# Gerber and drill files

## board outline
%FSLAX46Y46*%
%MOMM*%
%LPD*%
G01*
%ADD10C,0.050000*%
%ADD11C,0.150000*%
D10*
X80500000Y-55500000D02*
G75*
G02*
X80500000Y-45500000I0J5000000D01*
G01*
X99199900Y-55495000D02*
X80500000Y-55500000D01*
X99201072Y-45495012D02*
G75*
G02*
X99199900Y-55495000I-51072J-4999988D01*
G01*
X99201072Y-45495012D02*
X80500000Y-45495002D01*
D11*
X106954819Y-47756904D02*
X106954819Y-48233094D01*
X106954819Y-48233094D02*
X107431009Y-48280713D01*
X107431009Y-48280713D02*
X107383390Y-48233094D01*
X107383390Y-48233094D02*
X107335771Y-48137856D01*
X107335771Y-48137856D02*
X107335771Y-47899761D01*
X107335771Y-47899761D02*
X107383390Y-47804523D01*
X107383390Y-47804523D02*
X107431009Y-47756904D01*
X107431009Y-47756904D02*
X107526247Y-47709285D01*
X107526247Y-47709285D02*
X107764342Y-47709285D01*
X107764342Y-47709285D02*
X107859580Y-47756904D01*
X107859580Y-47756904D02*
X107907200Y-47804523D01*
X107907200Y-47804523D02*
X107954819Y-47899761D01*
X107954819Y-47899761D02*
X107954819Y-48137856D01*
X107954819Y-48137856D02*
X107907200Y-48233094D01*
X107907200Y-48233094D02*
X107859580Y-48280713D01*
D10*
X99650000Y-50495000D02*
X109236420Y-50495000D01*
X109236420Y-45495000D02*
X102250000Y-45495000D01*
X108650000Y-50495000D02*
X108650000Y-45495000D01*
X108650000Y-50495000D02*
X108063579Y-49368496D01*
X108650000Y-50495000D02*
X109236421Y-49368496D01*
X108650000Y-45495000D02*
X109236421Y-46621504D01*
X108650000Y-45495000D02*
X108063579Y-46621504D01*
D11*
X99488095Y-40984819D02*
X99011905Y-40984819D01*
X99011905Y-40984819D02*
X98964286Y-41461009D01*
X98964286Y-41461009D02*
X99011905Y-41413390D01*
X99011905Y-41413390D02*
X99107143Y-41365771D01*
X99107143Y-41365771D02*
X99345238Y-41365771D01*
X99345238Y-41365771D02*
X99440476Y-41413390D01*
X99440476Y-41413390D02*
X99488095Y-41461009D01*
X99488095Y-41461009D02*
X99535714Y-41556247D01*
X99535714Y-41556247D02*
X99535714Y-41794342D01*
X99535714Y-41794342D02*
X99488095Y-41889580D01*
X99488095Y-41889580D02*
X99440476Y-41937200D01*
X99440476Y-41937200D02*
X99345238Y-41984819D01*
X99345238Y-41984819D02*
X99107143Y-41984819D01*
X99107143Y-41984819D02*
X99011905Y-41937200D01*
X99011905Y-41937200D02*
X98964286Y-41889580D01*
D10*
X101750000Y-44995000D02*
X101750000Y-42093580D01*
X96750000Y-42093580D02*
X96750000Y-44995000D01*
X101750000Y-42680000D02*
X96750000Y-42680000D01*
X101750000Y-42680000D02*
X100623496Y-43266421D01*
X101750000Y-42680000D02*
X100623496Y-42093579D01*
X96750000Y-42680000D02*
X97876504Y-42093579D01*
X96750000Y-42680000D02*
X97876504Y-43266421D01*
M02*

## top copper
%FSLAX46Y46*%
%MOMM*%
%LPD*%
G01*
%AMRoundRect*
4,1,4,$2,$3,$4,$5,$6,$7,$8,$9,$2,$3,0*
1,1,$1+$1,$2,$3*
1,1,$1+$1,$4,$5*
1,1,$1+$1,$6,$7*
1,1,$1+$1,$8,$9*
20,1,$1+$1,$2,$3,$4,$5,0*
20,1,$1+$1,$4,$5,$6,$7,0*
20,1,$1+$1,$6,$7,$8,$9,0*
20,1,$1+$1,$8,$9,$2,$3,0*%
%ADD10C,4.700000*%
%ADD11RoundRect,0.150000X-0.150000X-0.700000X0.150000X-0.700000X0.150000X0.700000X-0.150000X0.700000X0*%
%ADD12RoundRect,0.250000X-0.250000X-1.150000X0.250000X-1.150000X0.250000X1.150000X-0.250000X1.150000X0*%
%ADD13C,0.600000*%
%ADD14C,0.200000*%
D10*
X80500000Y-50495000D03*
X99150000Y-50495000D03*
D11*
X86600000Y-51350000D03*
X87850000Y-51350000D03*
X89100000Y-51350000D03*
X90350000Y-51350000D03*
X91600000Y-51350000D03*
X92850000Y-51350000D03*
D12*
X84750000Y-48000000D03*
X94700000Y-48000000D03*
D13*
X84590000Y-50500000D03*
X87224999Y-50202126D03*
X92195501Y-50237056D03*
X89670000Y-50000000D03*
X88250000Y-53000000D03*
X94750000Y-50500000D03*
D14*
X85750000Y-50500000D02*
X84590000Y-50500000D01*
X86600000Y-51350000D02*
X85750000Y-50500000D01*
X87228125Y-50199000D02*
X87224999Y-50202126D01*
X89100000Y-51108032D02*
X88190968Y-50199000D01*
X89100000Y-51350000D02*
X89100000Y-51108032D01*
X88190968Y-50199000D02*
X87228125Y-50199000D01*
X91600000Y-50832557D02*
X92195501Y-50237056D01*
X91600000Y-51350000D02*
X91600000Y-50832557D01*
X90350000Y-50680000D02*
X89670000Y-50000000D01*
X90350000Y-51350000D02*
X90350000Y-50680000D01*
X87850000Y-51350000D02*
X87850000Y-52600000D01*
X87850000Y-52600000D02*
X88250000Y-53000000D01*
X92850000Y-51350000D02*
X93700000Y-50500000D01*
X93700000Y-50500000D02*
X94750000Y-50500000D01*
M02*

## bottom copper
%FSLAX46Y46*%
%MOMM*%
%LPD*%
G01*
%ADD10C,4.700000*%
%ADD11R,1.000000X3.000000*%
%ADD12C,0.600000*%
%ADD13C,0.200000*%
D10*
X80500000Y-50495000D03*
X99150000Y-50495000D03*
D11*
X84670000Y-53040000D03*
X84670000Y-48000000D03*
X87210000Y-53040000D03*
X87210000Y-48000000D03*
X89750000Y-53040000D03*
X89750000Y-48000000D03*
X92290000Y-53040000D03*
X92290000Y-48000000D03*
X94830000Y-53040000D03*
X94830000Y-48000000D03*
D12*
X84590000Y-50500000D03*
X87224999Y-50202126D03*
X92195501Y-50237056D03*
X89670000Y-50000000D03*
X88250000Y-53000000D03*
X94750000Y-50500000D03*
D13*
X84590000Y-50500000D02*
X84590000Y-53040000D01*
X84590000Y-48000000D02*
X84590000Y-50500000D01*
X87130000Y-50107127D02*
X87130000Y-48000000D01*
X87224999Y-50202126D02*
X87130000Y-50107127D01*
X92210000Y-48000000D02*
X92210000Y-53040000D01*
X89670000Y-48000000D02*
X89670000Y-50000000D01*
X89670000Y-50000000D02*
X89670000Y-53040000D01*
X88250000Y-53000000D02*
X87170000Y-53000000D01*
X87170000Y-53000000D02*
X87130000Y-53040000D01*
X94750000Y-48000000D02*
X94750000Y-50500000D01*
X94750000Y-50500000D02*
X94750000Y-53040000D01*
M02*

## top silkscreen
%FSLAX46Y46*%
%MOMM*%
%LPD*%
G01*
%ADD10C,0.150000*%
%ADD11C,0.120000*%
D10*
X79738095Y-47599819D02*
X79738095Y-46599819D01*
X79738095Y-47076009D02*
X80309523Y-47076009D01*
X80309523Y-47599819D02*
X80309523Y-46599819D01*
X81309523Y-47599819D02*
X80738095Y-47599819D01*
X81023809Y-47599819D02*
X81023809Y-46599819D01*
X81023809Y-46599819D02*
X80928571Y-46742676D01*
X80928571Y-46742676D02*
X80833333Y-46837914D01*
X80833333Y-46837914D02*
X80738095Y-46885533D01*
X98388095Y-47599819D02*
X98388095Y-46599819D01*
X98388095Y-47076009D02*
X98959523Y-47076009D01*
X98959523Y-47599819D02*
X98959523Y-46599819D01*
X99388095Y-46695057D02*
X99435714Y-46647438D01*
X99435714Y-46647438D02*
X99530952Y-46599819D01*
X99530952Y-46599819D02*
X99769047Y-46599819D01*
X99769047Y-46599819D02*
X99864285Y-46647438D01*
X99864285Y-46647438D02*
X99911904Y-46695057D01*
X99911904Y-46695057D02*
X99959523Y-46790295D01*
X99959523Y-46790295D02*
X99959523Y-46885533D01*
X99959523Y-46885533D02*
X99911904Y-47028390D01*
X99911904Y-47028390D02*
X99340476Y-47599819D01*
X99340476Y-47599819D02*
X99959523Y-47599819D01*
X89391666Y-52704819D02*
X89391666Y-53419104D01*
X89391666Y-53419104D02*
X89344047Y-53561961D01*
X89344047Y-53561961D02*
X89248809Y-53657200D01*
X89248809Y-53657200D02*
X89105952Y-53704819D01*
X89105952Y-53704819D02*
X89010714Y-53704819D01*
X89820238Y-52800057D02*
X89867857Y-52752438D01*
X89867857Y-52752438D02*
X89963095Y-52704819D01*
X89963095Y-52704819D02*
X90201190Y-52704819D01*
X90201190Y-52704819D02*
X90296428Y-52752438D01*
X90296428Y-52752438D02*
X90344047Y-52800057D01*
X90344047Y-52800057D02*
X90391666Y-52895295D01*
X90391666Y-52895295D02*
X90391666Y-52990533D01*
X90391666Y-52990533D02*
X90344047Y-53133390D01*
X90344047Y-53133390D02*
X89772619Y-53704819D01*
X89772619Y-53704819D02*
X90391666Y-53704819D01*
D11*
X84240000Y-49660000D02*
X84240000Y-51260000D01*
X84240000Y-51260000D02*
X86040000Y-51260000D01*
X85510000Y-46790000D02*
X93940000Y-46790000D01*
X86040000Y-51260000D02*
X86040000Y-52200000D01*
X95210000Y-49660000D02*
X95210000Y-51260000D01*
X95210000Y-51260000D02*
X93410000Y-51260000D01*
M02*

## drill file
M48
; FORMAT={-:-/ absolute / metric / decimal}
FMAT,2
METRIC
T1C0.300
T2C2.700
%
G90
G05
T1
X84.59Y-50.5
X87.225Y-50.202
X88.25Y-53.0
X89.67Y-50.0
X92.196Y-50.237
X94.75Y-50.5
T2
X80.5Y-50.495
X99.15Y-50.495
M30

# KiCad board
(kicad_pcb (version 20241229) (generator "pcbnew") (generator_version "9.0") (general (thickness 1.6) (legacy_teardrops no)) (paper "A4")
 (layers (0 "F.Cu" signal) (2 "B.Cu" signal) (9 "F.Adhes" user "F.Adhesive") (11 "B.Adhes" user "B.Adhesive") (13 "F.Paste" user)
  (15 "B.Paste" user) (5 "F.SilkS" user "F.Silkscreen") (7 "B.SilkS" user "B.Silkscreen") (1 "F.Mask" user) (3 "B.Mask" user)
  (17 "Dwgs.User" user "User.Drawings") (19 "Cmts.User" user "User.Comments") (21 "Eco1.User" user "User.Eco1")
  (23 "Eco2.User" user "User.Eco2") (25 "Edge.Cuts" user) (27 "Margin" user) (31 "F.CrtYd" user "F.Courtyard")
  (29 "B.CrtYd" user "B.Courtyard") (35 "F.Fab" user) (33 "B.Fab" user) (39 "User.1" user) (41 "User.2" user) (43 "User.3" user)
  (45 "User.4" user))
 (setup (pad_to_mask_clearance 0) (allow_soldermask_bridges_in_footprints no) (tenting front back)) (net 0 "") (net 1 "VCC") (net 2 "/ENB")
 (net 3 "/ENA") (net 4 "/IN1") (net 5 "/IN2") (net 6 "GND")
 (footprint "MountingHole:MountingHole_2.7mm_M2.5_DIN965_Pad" (layer "F.Cu") (at 80.5 50.495)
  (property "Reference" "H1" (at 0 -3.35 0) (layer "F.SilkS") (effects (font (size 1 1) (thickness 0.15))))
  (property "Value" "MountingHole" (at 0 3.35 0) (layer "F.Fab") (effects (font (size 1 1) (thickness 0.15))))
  (pad "1" thru_hole circle (at 0 0) (size 4.7 4.7) (drill 2.7) (layers "*.Cu" "*.Mask") (remove_unused_layers no)))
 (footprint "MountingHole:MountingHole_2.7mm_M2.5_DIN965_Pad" (layer "F.Cu") (at 99.15 50.495)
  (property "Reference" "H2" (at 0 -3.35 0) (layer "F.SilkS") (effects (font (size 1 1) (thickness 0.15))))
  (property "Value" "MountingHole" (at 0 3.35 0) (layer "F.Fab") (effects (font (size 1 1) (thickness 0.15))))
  (pad "1" thru_hole circle (at 0 0) (size 4.7 4.7) (drill 2.7) (layers "*.Cu" "*.Mask") (remove_unused_layers no)))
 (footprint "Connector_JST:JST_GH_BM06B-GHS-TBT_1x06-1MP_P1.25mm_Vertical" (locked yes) (layer "F.Cu") (at 89.725 49.4)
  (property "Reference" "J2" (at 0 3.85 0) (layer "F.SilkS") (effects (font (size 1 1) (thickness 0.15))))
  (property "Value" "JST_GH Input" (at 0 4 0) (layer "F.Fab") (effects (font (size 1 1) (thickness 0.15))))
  (fp_line (start -5.485 0.26) (end -5.485 1.86) (stroke (width 0.12) (type solid)) (layer "F.SilkS"))
  (fp_line (start -5.485 1.86) (end -3.685 1.86) (stroke (width 0.12) (type solid)) (layer "F.SilkS"))
  (fp_line (start -4.215 -2.61) (end 4.215 -2.61) (stroke (width 0.12) (type solid)) (layer "F.SilkS"))
  (fp_line (start -3.685 1.86) (end -3.685 2.8) (stroke (width 0.12) (type solid)) (layer "F.SilkS"))
  (fp_line (start 5.485 0.26) (end 5.485 1.86) (stroke (width 0.12) (type solid)) (layer "F.SilkS"))
  (fp_line (start 5.485 1.86) (end 3.685 1.86) (stroke (width 0.12) (type solid)) (layer "F.SilkS"))
  (pad "1" smd roundrect (at -3.125 1.95) (size 0.6 1.7) (layers "F.Cu" "F.Mask" "F.Paste") (roundrect_rratio 0.25) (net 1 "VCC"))
  (pad "2" smd roundrect (at -1.875 1.95) (size 0.6 1.7) (layers "F.Cu" "F.Mask" "F.Paste") (roundrect_rratio 0.25) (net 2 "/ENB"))
  (pad "3" smd roundrect (at -0.625 1.95) (size 0.6 1.7) (layers "F.Cu" "F.Mask" "F.Paste") (roundrect_rratio 0.25) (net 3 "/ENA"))
  (pad "4" smd roundrect (at 0.625 1.95) (size 0.6 1.7) (layers "F.Cu" "F.Mask" "F.Paste") (roundrect_rratio 0.25) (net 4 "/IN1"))
  (pad "5" smd roundrect (at 1.875 1.95) (size 0.6 1.7) (layers "F.Cu" "F.Mask" "F.Paste") (roundrect_rratio 0.25) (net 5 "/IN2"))
  (pad "6" smd roundrect (at 3.125 1.95) (size 0.6 1.7) (layers "F.Cu" "F.Mask" "F.Paste") (roundrect_rratio 0.25) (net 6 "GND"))
  (pad "MP" smd roundrect (at -4.975 -1.4) (size 1 2.8) (layers "F.Cu" "F.Mask" "F.Paste") (roundrect_rratio 0.25))
  (pad "MP" smd roundrect (at 4.975 -1.4) (size 1 2.8) (layers "F.Cu" "F.Mask" "F.Paste") (roundrect_rratio 0.25)))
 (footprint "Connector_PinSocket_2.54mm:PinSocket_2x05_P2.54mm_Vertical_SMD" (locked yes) (layer "B.Cu") (at 89.75 50.52 -90)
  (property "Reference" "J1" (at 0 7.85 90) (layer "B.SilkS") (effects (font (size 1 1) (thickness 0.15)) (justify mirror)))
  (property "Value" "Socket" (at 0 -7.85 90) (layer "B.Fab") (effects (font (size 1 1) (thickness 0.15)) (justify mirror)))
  (pad "1" smd rect (at 2.52 5.08 270) (size 3 1) (layers "B.Cu" "B.Mask" "B.Paste") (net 1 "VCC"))
  (pad "2" smd rect (at -2.52 5.08 270) (size 3 1) (layers "B.Cu" "B.Mask" "B.Paste") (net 1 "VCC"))
  (pad "3" smd rect (at 2.52 2.54 270) (size 3 1) (layers "B.Cu" "B.Mask" "B.Paste") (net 2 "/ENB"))
  (pad "4" smd rect (at -2.52 2.54 270) (size 3 1) (layers "B.Cu" "B.Mask" "B.Paste") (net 3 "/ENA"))
  (pad "5" smd rect (at 2.52 0 270) (size 3 1) (layers "B.Cu" "B.Mask" "B.Paste") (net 4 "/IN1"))
  (pad "6" smd rect (at -2.52 0 270) (size 3 1) (layers "B.Cu" "B.Mask" "B.Paste") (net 4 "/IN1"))
  (pad "7" smd rect (at 2.52 -2.54 270) (size 3 1) (layers "B.Cu" "B.Mask" "B.Paste") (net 5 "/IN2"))
  (pad "8" smd rect (at -2.52 -2.54 270) (size 3 1) (layers "B.Cu" "B.Mask" "B.Paste") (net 5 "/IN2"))
  (pad "9" smd rect (at 2.52 -5.08 270) (size 3 1) (layers "B.Cu" "B.Mask" "B.Paste") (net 6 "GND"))
  (pad "10" smd rect (at -2.52 -5.08 270) (size 3 1) (layers "B.Cu" "B.Mask" "B.Paste") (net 6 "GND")))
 (gr_arc (start 80.5 55.5) (mid 75.5 50.5) (end 80.5 45.5) (stroke (width 0.05) (type solid)) (layer "Edge.Cuts"))
 (gr_line (start 99.1999 55.495) (end 80.5 55.5) (stroke (width 0.05) (type default)) (layer "Edge.Cuts"))
 (gr_arc (start 99.201072 45.495012) (mid 104.150249 50.495586) (end 99.1999 55.495) (stroke (width 0.05) (type solid)) (layer "Edge.Cuts"))
 (gr_line (start 99.201072 45.495012) (end 80.5 45.495002) (stroke (width 0.05) (type default)) (layer "Edge.Cuts"))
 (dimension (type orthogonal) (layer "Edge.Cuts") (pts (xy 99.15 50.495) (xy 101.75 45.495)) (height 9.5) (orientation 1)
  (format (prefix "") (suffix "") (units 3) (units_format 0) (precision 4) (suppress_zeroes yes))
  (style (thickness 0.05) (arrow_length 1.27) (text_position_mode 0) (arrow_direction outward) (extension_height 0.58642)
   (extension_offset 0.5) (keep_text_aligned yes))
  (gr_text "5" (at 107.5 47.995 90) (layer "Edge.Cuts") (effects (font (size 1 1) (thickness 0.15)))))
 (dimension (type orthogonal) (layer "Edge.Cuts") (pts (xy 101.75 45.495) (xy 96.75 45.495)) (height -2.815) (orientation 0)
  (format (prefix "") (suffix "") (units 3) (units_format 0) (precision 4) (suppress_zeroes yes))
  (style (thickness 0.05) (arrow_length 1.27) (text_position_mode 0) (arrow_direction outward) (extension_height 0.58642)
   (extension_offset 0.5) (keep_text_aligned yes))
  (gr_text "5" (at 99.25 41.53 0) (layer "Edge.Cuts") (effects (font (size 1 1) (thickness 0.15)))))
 (segment (start 85.75 50.5) (end 84.59 50.5) (width 0.2) (layer "F.Cu") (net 1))
 (segment (start 86.6 51.35) (end 85.75 50.5) (width 0.2) (layer "F.Cu") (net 1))
 (via (at 84.59 50.5) (size 0.6) (drill 0.3) (layers "F.Cu" "B.Cu") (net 1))
 (segment (start 84.59 50.5) (end 84.59 53.04) (width 0.2) (layer "B.Cu") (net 1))
 (segment (start 84.59 48) (end 84.59 50.5) (width 0.2) (layer "B.Cu") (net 1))
 (segment (start 87.228125 50.199) (end 87.224999 50.202126) (width 0.2) (layer "F.Cu") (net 3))
 (segment (start 89.1 51.108032) (end 88.190968 50.199) (width 0.2) (layer "F.Cu") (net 3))
 (segment (start 89.1 51.35) (end 89.1 51.108032) (width 0.2) (layer "F.Cu") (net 3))
 (segment (start 88.190968 50.199) (end 87.228125 50.199) (width 0.2) (layer "F.Cu") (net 3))
 (via (at 87.224999 50.202126) (size 0.6) (drill 0.3) (layers "F.Cu" "B.Cu") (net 3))
 (segment (start 87.13 50.107127) (end 87.13 48) (width 0.2) (layer "B.Cu") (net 3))
 (segment (start 87.224999 50.202126) (end 87.13 50.107127) (width 0.2) (layer "B.Cu") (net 3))
 (segment (start 91.6 50.832557) (end 92.195501 50.237056) (width 0.2) (layer "F.Cu") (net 5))
 (segment (start 91.6 51.35) (end 91.6 50.832557) (width 0.2) (layer "F.Cu") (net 5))
 (via (at 92.195501 50.237056) (size 0.6) (drill 0.3) (layers "F.Cu" "B.Cu") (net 5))
 (segment (start 92.21 48) (end 92.21 53.04) (width 0.2) (layer "B.Cu") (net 5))
 (segment (start 90.35 50.68) (end 89.67 50) (width 0.2) (layer "F.Cu") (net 4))
 (segment (start 90.35 51.35) (end 90.35 50.68) (width 0.2) (layer "F.Cu") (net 4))
 (via (at 89.67 50) (size 0.6) (drill 0.3) (layers "F.Cu" "B.Cu") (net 4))
 (segment (start 89.67 48) (end 89.67 50) (width 0.2) (layer "B.Cu") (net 4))
 (segment (start 89.67 50) (end 89.67 53.04) (width 0.2) (layer "B.Cu") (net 4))
 (segment (start 87.85 51.35) (end 87.85 52.6) (width 0.2) (layer "F.Cu") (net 2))
 (segment (start 87.85 52.6) (end 88.25 53) (width 0.2) (layer "F.Cu") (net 2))
 (via (at 88.25 53) (size 0.6) (drill 0.3) (layers "F.Cu" "B.Cu") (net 2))
 (segment (start 88.25 53) (end 87.17 53) (width 0.2) (layer "B.Cu") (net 2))
 (segment (start 87.17 53) (end 87.13 53.04) (width 0.2) (layer "B.Cu") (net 2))
 (segment (start 92.85 51.35) (end 93.7 50.5) (width 0.2) (layer "F.Cu") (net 6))
 (segment (start 93.7 50.5) (end 94.75 50.5) (width 0.2) (layer "F.Cu") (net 6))
 (via (at 94.75 50.5) (size 0.6) (drill 0.3) (layers "F.Cu" "B.Cu") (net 6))
 (segment (start 94.75 48) (end 94.75 50.5) (width 0.2) (layer "B.Cu") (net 6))
 (segment (start 94.75 50.5) (end 94.75 53.04) (width 0.2) (layer "B.Cu") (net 6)))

